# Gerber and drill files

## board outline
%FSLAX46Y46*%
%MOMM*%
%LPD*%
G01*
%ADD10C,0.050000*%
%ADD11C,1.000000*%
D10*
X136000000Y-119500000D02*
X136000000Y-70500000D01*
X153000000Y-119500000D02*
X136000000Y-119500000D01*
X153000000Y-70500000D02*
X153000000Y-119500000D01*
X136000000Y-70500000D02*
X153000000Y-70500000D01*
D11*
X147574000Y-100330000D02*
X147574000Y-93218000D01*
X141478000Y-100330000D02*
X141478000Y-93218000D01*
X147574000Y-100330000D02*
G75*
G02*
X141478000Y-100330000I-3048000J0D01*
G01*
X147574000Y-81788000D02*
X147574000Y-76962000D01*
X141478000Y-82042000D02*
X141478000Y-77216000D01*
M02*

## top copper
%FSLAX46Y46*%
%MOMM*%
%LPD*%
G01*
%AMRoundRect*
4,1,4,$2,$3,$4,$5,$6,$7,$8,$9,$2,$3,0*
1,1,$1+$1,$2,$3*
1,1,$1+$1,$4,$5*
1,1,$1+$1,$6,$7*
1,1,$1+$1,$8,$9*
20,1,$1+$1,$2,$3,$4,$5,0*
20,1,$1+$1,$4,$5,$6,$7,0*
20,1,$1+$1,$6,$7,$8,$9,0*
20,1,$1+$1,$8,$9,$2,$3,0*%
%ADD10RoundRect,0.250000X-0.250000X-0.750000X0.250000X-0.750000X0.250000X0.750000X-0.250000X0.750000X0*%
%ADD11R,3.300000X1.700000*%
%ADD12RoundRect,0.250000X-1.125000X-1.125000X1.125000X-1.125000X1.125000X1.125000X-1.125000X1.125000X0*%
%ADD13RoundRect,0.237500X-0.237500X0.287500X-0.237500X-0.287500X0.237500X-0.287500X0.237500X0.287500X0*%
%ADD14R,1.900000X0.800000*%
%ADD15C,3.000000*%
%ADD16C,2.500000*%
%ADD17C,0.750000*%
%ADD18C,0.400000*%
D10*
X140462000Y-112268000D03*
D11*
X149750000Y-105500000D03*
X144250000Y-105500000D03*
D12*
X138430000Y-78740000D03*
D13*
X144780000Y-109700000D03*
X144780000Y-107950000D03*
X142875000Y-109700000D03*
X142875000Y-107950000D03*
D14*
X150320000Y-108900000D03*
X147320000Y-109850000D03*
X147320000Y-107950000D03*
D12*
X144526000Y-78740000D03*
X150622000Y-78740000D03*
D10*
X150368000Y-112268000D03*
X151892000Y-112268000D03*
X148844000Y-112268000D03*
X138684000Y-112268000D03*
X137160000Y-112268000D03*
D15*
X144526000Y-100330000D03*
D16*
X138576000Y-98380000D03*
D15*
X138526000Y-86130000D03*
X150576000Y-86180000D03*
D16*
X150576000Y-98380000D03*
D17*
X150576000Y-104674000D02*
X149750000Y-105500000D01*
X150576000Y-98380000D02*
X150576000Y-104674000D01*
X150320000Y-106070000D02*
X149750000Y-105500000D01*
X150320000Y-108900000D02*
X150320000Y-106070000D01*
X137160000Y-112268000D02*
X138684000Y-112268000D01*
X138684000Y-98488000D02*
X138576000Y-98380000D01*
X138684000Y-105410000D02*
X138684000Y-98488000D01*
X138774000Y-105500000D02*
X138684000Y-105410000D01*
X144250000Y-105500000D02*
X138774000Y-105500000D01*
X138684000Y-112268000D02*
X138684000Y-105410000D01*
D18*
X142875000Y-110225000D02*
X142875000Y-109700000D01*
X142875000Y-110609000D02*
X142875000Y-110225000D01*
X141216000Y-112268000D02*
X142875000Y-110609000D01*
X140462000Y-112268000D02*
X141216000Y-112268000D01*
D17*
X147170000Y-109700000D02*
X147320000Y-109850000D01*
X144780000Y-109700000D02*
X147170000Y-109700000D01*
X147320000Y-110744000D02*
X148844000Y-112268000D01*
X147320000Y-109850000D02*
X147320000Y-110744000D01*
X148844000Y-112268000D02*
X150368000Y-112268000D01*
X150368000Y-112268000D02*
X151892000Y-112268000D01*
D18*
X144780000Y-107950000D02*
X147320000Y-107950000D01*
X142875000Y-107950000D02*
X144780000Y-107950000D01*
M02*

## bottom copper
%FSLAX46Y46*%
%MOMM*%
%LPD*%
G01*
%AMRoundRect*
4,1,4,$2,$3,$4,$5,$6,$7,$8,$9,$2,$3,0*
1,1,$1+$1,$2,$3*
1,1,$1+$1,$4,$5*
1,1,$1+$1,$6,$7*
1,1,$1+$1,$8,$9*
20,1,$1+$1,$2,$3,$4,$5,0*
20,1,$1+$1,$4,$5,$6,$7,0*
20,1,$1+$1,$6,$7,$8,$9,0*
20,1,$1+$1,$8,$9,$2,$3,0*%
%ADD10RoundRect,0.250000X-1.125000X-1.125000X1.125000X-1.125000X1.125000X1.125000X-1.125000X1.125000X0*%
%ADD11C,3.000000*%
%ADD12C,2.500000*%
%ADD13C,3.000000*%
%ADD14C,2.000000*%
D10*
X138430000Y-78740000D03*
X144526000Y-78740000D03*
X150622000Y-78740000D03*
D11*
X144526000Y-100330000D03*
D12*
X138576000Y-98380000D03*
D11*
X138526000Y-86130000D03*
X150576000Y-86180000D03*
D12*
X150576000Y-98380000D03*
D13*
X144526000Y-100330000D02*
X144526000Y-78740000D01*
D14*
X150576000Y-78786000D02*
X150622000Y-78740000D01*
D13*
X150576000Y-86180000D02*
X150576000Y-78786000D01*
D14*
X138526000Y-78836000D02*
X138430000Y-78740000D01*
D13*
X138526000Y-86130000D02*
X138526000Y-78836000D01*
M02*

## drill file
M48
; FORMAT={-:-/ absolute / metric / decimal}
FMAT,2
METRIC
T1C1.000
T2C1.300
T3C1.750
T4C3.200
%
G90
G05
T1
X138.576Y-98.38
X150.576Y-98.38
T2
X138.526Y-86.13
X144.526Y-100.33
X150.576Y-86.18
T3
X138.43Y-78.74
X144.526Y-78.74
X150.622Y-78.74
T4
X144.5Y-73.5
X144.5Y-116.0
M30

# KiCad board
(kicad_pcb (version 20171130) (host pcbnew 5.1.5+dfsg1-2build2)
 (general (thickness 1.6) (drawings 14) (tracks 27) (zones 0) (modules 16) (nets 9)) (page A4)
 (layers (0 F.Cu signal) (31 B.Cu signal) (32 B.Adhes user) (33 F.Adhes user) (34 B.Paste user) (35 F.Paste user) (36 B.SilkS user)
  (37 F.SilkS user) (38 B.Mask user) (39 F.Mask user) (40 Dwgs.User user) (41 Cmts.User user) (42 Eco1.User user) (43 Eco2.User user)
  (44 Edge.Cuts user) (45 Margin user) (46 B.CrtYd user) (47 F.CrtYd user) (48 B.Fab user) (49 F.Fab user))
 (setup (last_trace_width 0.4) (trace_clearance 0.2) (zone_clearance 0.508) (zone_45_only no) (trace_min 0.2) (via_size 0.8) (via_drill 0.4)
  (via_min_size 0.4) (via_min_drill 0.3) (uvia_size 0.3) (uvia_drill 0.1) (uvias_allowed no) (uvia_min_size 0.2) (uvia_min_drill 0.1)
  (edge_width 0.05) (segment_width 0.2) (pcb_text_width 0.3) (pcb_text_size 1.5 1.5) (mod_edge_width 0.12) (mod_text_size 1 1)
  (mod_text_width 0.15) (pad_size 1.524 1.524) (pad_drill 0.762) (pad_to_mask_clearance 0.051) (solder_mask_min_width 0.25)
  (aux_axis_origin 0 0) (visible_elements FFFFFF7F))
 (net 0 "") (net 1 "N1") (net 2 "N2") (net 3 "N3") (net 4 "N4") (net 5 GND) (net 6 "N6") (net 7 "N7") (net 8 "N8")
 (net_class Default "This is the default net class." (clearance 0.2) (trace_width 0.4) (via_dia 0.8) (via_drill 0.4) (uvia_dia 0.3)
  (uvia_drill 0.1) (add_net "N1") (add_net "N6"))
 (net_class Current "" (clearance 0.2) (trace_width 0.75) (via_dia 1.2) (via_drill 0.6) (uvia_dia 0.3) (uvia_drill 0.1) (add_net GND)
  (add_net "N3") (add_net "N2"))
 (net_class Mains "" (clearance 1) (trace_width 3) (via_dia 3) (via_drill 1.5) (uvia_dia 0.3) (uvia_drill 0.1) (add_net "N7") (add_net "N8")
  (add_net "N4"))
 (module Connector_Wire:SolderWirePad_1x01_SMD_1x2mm (layer F.Cu) (at 140.462 112.268)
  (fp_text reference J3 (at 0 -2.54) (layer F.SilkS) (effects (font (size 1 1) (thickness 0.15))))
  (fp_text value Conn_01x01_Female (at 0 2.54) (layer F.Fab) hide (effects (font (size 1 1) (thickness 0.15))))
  (pad 1 smd roundrect (at 0 0) (size 1 2) (layers F.Cu F.Paste F.Mask) (roundrect_rratio 0.25) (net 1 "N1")))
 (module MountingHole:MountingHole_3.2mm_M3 (layer F.Cu) (at 144.5 116)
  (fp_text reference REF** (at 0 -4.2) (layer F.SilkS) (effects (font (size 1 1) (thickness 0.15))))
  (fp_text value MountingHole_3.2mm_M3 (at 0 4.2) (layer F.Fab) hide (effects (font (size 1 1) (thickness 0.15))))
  (pad 1 np_thru_hole circle (at 0 0) (size 3.2 3.2) (drill 3.2) (layers *.Cu *.Mask)))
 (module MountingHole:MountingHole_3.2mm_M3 (layer F.Cu) (at 144.5 73.5)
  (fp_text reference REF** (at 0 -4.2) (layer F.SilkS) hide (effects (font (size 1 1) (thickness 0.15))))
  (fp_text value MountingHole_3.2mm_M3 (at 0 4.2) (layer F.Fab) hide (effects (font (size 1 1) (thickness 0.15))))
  (pad 1 np_thru_hole circle (at 0 0) (size 3.2 3.2) (drill 3.2) (layers *.Cu *.Mask)))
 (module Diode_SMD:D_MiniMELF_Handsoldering (layer F.Cu) (at 147 105.5)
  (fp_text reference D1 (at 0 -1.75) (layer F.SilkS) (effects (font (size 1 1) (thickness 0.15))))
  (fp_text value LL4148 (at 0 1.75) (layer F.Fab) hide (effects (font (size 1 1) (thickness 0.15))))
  (pad 2 smd rect (at 2.75 0) (size 3.3 1.7) (layers F.Cu F.Paste F.Mask) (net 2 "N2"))
  (pad 1 smd rect (at -2.75 0) (size 3.3 1.7) (layers F.Cu F.Paste F.Mask) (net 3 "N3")))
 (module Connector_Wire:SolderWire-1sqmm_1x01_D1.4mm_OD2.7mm (layer F.Cu) (at 138.43 78.74)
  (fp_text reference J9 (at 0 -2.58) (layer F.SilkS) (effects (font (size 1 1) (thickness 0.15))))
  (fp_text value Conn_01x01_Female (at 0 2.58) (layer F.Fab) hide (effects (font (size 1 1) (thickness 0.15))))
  (pad 1 thru_hole roundrect (at 0 0) (size 2.75 2.75) (drill 1.75) (layers *.Cu *.Mask) (roundrect_rratio 0.090909) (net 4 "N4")))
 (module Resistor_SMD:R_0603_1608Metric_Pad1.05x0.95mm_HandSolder (layer F.Cu) (at 144.78 108.825 270)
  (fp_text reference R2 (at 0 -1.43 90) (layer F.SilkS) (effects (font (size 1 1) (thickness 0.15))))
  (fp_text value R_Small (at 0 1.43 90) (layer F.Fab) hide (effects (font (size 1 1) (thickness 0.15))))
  (pad 2 smd roundrect (at 0.875 0 270) (size 1.05 0.95) (layers F.Cu F.Paste F.Mask) (roundrect_rratio 0.25) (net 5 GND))
  (pad 1 smd roundrect (at -0.875 0 270) (size 1.05 0.95) (layers F.Cu F.Paste F.Mask) (roundrect_rratio 0.25) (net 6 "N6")))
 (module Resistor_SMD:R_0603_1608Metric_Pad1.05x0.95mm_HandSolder (layer F.Cu) (at 142.875 108.825 270)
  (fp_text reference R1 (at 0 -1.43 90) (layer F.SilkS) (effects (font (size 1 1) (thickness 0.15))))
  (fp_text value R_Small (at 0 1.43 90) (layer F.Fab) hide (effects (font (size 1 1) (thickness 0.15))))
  (pad 2 smd roundrect (at 0.875 0 270) (size 1.05 0.95) (layers F.Cu F.Paste F.Mask) (roundrect_rratio 0.25) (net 1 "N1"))
  (pad 1 smd roundrect (at -0.875 0 270) (size 1.05 0.95) (layers F.Cu F.Paste F.Mask) (roundrect_rratio 0.25) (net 6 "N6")))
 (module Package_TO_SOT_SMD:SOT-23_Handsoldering (layer F.Cu) (at 148.82 108.9)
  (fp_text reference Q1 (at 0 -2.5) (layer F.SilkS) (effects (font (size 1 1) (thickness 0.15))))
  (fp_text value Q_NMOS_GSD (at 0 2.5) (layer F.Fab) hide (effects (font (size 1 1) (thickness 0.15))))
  (pad 3 smd rect (at 1.5 0) (size 1.9 0.8) (layers F.Cu F.Paste F.Mask) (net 2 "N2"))
  (pad 2 smd rect (at -1.5 0.95) (size 1.9 0.8) (layers F.Cu F.Paste F.Mask) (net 5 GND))
  (pad 1 smd rect (at -1.5 -0.95) (size 1.9 0.8) (layers F.Cu F.Paste F.Mask) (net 6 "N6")))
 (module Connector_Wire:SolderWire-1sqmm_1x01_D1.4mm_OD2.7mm (layer F.Cu) (at 144.526 78.74)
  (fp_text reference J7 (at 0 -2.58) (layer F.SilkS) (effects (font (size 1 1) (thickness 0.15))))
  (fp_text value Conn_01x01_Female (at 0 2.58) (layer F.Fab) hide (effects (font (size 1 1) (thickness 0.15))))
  (pad 1 thru_hole roundrect (at 0 0) (size 2.75 2.75) (drill 1.75) (layers *.Cu *.Mask) (roundrect_rratio 0.090909) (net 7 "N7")))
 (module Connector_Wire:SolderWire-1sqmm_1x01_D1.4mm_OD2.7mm (layer F.Cu) (at 150.622 78.74)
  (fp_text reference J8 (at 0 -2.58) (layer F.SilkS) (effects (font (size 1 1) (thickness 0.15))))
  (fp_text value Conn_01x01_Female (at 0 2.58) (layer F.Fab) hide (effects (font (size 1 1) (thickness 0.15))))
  (pad 1 thru_hole roundrect (at 0 0) (size 2.75 2.75) (drill 1.75) (layers *.Cu *.Mask) (roundrect_rratio 0.090909) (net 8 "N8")))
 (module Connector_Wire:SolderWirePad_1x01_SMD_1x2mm (layer F.Cu) (at 150.368 112.268)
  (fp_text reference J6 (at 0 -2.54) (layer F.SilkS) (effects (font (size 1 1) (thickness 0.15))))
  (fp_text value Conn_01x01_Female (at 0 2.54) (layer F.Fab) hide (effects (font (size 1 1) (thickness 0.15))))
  (pad 1 smd roundrect (at 0 0) (size 1 2) (layers F.Cu F.Paste F.Mask) (roundrect_rratio 0.25) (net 5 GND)))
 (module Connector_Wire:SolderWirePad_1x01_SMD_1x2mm (layer F.Cu) (at 151.892 112.268)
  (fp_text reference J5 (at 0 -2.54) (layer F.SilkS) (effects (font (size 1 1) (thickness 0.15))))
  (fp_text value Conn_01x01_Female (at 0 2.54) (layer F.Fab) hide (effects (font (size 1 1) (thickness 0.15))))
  (pad 1 smd roundrect (at 0 0) (size 1 2) (layers F.Cu F.Paste F.Mask) (roundrect_rratio 0.25) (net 5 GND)))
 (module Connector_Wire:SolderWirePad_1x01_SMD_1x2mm (layer F.Cu) (at 148.844 112.268)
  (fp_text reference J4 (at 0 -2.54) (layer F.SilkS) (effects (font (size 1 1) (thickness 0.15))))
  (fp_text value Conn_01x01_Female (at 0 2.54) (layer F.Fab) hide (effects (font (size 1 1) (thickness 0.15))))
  (pad 1 smd roundrect (at 0 0) (size 1 2) (layers F.Cu F.Paste F.Mask) (roundrect_rratio 0.25) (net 5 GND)))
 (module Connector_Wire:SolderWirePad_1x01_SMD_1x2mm (layer F.Cu) (at 138.684 112.268)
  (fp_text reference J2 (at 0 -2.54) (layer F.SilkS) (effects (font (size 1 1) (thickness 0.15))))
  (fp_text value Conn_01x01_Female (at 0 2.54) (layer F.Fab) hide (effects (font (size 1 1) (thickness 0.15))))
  (pad 1 smd roundrect (at 0 0) (size 1 2) (layers F.Cu F.Paste F.Mask) (roundrect_rratio 0.25) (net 3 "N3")))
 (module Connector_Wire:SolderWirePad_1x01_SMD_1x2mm (layer F.Cu) (at 137.16 112.268)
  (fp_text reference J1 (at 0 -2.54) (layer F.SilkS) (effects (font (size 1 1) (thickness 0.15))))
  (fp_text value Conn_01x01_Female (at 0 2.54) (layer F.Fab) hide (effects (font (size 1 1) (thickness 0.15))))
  (pad 1 smd roundrect (at 0 0) (size 1 2) (layers F.Cu F.Paste F.Mask) (roundrect_rratio 0.25) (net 3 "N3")))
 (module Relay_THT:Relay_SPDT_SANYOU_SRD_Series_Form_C (layer F.Cu) (at 144.526 100.33 90)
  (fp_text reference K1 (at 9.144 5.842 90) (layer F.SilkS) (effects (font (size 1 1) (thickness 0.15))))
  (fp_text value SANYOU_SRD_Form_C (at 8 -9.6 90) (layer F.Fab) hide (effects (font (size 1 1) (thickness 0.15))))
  (pad 1 thru_hole circle (at 0 0 180) (size 3 3) (drill 1.3) (layers *.Cu *.Mask) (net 7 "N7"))
  (pad 5 thru_hole circle (at 1.95 -5.95 180) (size 2.5 2.5) (drill 1) (layers *.Cu *.Mask) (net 3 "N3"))
  (pad 4 thru_hole circle (at 14.2 -6 180) (size 3 3) (drill 1.3) (layers *.Cu *.Mask) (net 4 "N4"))
  (pad 3 thru_hole circle (at 14.15 6.05 180) (size 3 3) (drill 1.3) (layers *.Cu *.Mask) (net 8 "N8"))
  (pad 2 thru_hole circle (at 1.95 6.05 180) (size 2.5 2.5) (drill 1) (layers *.Cu *.Mask) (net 2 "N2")))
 (gr_line (start 136 119.5) (end 136 70.5) (layer Edge.Cuts) (width 0.05))
 (gr_line (start 153 119.5) (end 136 119.5) (layer Edge.Cuts) (width 0.05))
 (gr_line (start 153 70.5) (end 153 119.5) (layer Edge.Cuts) (width 0.05))
 (gr_line (start 136 70.5) (end 153 70.5) (layer Edge.Cuts) (width 0.05))
 (gr_line (start 147.574 100.33) (end 147.574 93.218) (layer Edge.Cuts) (width 1))
 (gr_line (start 141.478 100.33) (end 141.478 93.218) (layer Edge.Cuts) (width 1))
 (gr_arc (start 144.526 100.33) (end 141.478 100.33) (angle -180) (layer Edge.Cuts) (width 1))
 (gr_line (start 147.574 81.788) (end 147.574 76.962) (layer Edge.Cuts) (width 1))
 (gr_line (start 141.478 82.042) (end 141.478 77.216) (layer Edge.Cuts) (width 1))
 (segment (start 150.576 104.674) (end 149.75 105.5) (width 0.75) (layer F.Cu) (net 2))
 (segment (start 150.576 98.38) (end 150.576 104.674) (width 0.75) (layer F.Cu) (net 2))
 (segment (start 150.32 106.07) (end 149.75 105.5) (width 0.75) (layer F.Cu) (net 2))
 (segment (start 150.32 108.9) (end 150.32 106.07) (width 0.75) (layer F.Cu) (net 2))
 (segment (start 137.16 112.268) (end 138.684 112.268) (width 0.75) (layer F.Cu) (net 3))
 (segment (start 138.684 98.488) (end 138.576 98.38) (width 0.75) (layer F.Cu) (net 3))
 (segment (start 138.684 105.41) (end 138.684 98.488) (width 0.75) (layer F.Cu) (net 3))
 (segment (start 138.774 105.5) (end 138.684 105.41) (width 0.75) (layer F.Cu) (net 3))
 (segment (start 144.25 105.5) (end 138.774 105.5) (width 0.75) (layer F.Cu) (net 3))
 (segment (start 138.684 112.268) (end 138.684 105.41) (width 0.75) (layer F.Cu) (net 3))
 (segment (start 142.875 110.225) (end 142.875 109.7) (width 0.4) (layer F.Cu) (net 1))
 (segment (start 142.875 110.609) (end 142.875 110.225) (width 0.4) (layer F.Cu) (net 1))
 (segment (start 141.216 112.268) (end 142.875 110.609) (width 0.4) (layer F.Cu) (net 1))
 (segment (start 140.462 112.268) (end 141.216 112.268) (width 0.4) (layer F.Cu) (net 1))
 (segment (start 147.17 109.7) (end 147.32 109.85) (width 0.75) (layer F.Cu) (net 5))
 (segment (start 144.78 109.7) (end 147.17 109.7) (width 0.75) (layer F.Cu) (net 5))
 (segment (start 147.32 110.744) (end 148.844 112.268) (width 0.75) (layer F.Cu) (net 5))
 (segment (start 147.32 109.85) (end 147.32 110.744) (width 0.75) (layer F.Cu) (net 5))
 (segment (start 148.844 112.268) (end 150.368 112.268) (width 0.75) (layer F.Cu) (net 5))
 (segment (start 150.368 112.268) (end 151.892 112.268) (width 0.75) (layer F.Cu) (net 5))
 (segment (start 144.526 100.33) (end 144.526 78.74) (width 3) (layer B.Cu) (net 7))
 (segment (start 150.576 78.786) (end 150.622 78.74) (width 2) (layer B.Cu) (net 8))
 (segment (start 150.576 86.18) (end 150.576 78.786) (width 3) (layer B.Cu) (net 8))
 (segment (start 144.78 107.95) (end 147.32 107.95) (width 0.4) (layer F.Cu) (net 6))
 (segment (start 142.875 107.95) (end 144.78 107.95) (width 0.4) (layer F.Cu) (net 6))
 (segment (start 138.526 78.836) (end 138.43 78.74) (width 2) (layer B.Cu) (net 4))
 (segment (start 138.526 86.13) (end 138.526 78.836) (width 3) (layer B.Cu) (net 4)))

